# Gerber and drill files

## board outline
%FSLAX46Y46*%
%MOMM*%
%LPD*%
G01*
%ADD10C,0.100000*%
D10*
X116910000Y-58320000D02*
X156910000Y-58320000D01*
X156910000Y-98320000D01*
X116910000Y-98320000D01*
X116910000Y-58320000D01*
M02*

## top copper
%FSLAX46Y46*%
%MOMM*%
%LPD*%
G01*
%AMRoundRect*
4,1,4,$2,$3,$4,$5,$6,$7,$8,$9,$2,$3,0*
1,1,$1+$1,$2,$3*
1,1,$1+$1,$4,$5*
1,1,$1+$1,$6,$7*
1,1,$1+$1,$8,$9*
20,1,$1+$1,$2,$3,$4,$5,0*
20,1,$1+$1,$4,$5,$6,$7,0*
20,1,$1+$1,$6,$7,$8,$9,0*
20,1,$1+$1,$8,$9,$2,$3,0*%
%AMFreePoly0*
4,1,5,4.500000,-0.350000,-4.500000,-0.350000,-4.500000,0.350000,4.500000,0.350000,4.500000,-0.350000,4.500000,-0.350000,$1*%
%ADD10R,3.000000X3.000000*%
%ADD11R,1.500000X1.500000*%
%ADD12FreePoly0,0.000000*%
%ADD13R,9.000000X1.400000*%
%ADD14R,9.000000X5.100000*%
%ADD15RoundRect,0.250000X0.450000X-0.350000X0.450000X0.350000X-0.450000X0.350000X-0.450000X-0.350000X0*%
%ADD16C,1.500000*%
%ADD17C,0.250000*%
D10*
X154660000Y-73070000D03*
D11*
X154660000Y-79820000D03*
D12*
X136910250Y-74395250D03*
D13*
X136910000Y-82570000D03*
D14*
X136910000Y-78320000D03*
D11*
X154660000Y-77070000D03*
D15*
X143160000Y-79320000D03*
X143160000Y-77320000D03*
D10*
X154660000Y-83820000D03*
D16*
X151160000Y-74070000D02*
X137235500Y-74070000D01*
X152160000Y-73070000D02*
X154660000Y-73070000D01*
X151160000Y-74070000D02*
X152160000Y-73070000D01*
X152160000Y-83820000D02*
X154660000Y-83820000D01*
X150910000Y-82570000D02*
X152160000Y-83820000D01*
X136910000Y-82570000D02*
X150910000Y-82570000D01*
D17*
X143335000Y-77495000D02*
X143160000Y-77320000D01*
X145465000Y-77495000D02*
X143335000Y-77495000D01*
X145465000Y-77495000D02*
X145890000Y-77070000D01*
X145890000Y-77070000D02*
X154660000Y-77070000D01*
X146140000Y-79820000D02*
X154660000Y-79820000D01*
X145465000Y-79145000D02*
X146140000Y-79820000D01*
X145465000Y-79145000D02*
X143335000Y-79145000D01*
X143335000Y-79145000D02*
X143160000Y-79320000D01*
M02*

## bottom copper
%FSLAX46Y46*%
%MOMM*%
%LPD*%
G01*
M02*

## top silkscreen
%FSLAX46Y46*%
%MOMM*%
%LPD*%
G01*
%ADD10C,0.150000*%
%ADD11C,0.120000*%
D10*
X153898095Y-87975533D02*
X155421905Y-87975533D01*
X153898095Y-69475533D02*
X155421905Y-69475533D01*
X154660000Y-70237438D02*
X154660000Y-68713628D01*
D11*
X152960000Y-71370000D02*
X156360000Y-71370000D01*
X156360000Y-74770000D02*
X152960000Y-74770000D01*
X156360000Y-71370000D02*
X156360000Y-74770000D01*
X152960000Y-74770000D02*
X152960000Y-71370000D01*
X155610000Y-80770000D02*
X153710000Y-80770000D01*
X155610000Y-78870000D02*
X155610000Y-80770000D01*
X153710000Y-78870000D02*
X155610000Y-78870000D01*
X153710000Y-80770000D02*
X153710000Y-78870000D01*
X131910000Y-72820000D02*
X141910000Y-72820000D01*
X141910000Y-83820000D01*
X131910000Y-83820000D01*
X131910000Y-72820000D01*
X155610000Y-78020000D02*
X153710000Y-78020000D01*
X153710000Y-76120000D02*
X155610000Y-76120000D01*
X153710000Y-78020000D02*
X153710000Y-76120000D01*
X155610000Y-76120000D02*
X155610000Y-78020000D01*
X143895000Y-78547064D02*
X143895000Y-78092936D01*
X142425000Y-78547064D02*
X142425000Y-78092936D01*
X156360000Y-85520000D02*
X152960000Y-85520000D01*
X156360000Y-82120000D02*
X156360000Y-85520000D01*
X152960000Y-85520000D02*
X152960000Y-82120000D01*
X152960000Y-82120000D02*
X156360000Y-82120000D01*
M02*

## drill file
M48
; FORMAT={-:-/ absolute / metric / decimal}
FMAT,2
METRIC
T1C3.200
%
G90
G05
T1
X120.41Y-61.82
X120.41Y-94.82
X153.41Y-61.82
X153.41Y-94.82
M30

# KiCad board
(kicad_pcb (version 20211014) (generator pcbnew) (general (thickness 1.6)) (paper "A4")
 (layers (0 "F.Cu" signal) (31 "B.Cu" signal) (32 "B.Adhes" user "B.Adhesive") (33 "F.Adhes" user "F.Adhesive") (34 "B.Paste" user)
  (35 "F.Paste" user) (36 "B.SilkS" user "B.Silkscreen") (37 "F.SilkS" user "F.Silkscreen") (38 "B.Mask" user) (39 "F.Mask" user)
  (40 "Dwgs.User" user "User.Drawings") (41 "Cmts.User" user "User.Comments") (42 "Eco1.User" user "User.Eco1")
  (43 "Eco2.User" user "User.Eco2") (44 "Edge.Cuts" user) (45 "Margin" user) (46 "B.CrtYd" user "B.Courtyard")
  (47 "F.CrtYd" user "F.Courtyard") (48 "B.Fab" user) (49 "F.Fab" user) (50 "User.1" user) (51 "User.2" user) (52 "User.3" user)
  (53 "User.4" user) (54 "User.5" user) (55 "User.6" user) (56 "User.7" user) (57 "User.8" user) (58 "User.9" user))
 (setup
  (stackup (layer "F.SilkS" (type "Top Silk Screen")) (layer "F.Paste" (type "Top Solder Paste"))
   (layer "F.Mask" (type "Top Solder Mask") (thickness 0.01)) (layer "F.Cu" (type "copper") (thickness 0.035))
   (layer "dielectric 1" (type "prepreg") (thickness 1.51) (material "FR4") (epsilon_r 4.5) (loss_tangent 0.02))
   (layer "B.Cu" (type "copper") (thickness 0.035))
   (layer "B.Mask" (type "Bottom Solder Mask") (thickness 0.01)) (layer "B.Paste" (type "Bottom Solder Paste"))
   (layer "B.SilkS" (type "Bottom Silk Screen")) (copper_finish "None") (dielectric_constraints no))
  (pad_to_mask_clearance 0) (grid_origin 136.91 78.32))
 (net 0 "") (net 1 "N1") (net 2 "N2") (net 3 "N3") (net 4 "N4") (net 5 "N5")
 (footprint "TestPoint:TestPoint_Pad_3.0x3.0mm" (layer "F.Cu") (at 154.66 73.07)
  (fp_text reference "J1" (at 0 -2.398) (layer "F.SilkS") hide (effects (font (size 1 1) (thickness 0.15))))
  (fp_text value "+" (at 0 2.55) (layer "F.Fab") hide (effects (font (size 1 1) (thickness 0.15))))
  (fp_line (start -1.7 -1.7) (end 1.7 -1.7) (layer "F.SilkS") (width 0.12))
  (fp_line (start 1.7 1.7) (end -1.7 1.7) (layer "F.SilkS") (width 0.12))
  (fp_line (start 1.7 -1.7) (end 1.7 1.7) (layer "F.SilkS") (width 0.12))
  (fp_line (start -1.7 1.7) (end -1.7 -1.7) (layer "F.SilkS") (width 0.12))
  (pad "1" smd rect (at 0 0) (size 3 3) (layers "F.Cu" "F.Mask") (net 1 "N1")))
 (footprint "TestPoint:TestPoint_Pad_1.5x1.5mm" (layer "F.Cu") (at 154.66 79.82)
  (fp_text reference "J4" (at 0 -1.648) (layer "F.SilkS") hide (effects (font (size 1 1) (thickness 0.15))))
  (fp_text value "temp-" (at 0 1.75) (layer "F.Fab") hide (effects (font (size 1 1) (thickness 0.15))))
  (fp_line (start 0.95 0.95) (end -0.95 0.95) (layer "F.SilkS") (width 0.12))
  (fp_line (start 0.95 -0.95) (end 0.95 0.95) (layer "F.SilkS") (width 0.12))
  (fp_line (start -0.95 -0.95) (end 0.95 -0.95) (layer "F.SilkS") (width 0.12))
  (fp_line (start -0.95 0.95) (end -0.95 -0.95) (layer "F.SilkS") (width 0.12))
  (pad "1" smd rect (at 0 0) (size 1.5 1.5) (layers "F.Cu" "F.Mask") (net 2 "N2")))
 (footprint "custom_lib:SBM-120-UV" (layer "F.Cu") (at 136.91 78.32)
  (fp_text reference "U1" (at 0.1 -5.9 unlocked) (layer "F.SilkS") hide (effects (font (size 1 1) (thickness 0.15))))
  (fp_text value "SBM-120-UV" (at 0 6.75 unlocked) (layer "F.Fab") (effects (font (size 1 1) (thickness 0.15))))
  (fp_rect (start -5 -5.5) (end 5 5.5) (layer "F.SilkS") (width 0.12) (fill none))
  (pad "1" smd custom (at 0.00025 -3.92475) (size 9 0.7) (layers "F.Cu" "F.Paste" "F.Mask") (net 1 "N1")
   (options (clearance outline) (anchor rect)) (primitives))
  (pad "2" smd rect (at 0 4.25) (size 9 1.4) (layers "F.Cu" "F.Paste" "F.Mask") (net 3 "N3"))
  (pad "3" smd rect (at 0 0) (size 9 5.1) (layers "F.Cu" "F.Paste" "F.Mask") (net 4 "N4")))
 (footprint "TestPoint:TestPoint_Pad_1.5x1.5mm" (layer "F.Cu") (at 154.66 77.07)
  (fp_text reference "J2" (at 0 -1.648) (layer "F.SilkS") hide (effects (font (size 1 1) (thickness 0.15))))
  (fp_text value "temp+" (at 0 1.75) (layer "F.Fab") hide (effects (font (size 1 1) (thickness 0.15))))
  (fp_line (start 0.95 0.95) (end -0.95 0.95) (layer "F.SilkS") (width 0.12))
  (fp_line (start -0.95 -0.95) (end 0.95 -0.95) (layer "F.SilkS") (width 0.12))
  (fp_line (start -0.95 0.95) (end -0.95 -0.95) (layer "F.SilkS") (width 0.12))
  (fp_line (start 0.95 -0.95) (end 0.95 0.95) (layer "F.SilkS") (width 0.12))
  (pad "1" smd rect (at 0 0) (size 1.5 1.5) (layers "F.Cu" "F.Mask") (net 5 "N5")))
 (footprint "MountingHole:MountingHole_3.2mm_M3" (layer "F.Cu") (at 153.41 61.82)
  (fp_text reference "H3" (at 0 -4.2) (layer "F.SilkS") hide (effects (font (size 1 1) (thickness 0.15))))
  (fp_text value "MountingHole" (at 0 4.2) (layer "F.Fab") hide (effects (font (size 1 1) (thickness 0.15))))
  (pad "" np_thru_hole circle (at 0 0) (size 3.2 3.2) (drill 3.2) (layers *.Cu *.Mask)))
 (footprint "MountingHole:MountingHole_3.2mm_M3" (layer "F.Cu") (at 120.41 94.82)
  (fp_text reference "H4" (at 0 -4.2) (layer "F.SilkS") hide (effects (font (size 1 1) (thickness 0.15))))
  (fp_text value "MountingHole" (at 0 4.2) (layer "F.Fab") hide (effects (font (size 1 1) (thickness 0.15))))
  (pad "" np_thru_hole circle (at 0 0) (size 3.2 3.2) (drill 3.2) (layers *.Cu *.Mask)))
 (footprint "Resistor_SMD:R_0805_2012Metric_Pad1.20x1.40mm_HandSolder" (layer "F.Cu") (at 143.16 78.32 90)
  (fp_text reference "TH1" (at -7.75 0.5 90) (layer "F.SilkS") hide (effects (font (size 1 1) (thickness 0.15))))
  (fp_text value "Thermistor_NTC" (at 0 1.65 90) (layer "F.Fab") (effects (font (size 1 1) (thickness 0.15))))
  (fp_line (start -0.227064 0.735) (end 0.227064 0.735) (layer "F.SilkS") (width 0.12))
  (fp_line (start -0.227064 -0.735) (end 0.227064 -0.735) (layer "F.SilkS") (width 0.12))
  (pad "1" smd roundrect (at -1 0 90) (size 1.2 1.4) (layers "F.Cu" "F.Paste" "F.Mask") (roundrect_rratio 0.2083333333) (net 2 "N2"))
  (pad "2" smd roundrect (at 1 0 90) (size 1.2 1.4) (layers "F.Cu" "F.Paste" "F.Mask") (roundrect_rratio 0.2083333333) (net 5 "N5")))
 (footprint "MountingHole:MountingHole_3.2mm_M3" (layer "F.Cu") (at 153.41 94.82)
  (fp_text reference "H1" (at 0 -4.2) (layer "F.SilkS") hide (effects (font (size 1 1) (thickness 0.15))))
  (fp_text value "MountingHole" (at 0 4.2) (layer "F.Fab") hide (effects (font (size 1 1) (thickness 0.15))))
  (pad "" np_thru_hole circle (at 0 0) (size 3.2 3.2) (drill 3.2) (layers *.Cu *.Mask)))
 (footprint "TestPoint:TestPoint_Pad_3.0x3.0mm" (layer "F.Cu") (at 154.66 83.82)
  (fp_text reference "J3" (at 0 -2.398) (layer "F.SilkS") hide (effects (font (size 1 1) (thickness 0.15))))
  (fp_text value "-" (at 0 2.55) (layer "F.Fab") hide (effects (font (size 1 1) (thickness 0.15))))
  (fp_line (start 1.7 1.7) (end -1.7 1.7) (layer "F.SilkS") (width 0.12))
  (fp_line (start 1.7 -1.7) (end 1.7 1.7) (layer "F.SilkS") (width 0.12))
  (fp_line (start -1.7 1.7) (end -1.7 -1.7) (layer "F.SilkS") (width 0.12))
  (fp_line (start -1.7 -1.7) (end 1.7 -1.7) (layer "F.SilkS") (width 0.12))
  (pad "1" smd rect (at 0 0) (size 3 3) (layers "F.Cu" "F.Mask") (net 3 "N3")))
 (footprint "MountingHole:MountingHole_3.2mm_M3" (layer "F.Cu") (at 120.41 61.82)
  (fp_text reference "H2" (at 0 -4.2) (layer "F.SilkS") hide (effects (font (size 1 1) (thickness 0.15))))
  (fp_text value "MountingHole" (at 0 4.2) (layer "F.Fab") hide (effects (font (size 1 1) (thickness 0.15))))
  (pad "" np_thru_hole circle (at 0 0) (size 3.2 3.2) (drill 3.2) (layers *.Cu *.Mask)))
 (gr_rect (start 116.91 58.32) (end 156.91 98.32) (layer "Edge.Cuts") (width 0.1) (fill none))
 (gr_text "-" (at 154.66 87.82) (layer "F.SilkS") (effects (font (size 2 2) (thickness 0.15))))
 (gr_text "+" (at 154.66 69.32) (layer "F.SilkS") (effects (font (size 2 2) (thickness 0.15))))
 (segment (start 151.16 74.07) (end 137.2355 74.07) (width 1.5) (layer "F.Cu") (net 1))
 (segment (start 152.16 73.07) (end 154.66 73.07) (width 1.5) (layer "F.Cu") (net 1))
 (segment (start 151.16 74.07) (end 152.16 73.07) (width 1.5) (layer "F.Cu") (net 1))
 (segment (start 152.16 83.82) (end 154.66 83.82) (width 1.5) (layer "F.Cu") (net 3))
 (segment (start 150.91 82.57) (end 152.16 83.82) (width 1.5) (layer "F.Cu") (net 3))
 (segment (start 136.91 82.57) (end 150.91 82.57) (width 1.5) (layer "F.Cu") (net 3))
 (segment (start 143.335 77.495) (end 143.16 77.32) (width 0.25) (layer "F.Cu") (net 5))
 (segment (start 145.465 77.495) (end 143.335 77.495) (width 0.25) (layer "F.Cu") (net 5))
 (segment (start 145.465 77.495) (end 145.89 77.07) (width 0.25) (layer "F.Cu") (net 5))
 (segment (start 145.89 77.07) (end 154.66 77.07) (width 0.25) (layer "F.Cu") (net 5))
 (segment (start 146.14 79.82) (end 154.66 79.82) (width 0.25) (layer "F.Cu") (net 2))
 (segment (start 145.465 79.145) (end 146.14 79.82) (width 0.25) (layer "F.Cu") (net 2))
 (segment (start 145.465 79.145) (end 143.335 79.145) (width 0.25) (layer "F.Cu") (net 2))
 (segment (start 143.335 79.145) (end 143.16 79.32) (width 0.25) (layer "F.Cu") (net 2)))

